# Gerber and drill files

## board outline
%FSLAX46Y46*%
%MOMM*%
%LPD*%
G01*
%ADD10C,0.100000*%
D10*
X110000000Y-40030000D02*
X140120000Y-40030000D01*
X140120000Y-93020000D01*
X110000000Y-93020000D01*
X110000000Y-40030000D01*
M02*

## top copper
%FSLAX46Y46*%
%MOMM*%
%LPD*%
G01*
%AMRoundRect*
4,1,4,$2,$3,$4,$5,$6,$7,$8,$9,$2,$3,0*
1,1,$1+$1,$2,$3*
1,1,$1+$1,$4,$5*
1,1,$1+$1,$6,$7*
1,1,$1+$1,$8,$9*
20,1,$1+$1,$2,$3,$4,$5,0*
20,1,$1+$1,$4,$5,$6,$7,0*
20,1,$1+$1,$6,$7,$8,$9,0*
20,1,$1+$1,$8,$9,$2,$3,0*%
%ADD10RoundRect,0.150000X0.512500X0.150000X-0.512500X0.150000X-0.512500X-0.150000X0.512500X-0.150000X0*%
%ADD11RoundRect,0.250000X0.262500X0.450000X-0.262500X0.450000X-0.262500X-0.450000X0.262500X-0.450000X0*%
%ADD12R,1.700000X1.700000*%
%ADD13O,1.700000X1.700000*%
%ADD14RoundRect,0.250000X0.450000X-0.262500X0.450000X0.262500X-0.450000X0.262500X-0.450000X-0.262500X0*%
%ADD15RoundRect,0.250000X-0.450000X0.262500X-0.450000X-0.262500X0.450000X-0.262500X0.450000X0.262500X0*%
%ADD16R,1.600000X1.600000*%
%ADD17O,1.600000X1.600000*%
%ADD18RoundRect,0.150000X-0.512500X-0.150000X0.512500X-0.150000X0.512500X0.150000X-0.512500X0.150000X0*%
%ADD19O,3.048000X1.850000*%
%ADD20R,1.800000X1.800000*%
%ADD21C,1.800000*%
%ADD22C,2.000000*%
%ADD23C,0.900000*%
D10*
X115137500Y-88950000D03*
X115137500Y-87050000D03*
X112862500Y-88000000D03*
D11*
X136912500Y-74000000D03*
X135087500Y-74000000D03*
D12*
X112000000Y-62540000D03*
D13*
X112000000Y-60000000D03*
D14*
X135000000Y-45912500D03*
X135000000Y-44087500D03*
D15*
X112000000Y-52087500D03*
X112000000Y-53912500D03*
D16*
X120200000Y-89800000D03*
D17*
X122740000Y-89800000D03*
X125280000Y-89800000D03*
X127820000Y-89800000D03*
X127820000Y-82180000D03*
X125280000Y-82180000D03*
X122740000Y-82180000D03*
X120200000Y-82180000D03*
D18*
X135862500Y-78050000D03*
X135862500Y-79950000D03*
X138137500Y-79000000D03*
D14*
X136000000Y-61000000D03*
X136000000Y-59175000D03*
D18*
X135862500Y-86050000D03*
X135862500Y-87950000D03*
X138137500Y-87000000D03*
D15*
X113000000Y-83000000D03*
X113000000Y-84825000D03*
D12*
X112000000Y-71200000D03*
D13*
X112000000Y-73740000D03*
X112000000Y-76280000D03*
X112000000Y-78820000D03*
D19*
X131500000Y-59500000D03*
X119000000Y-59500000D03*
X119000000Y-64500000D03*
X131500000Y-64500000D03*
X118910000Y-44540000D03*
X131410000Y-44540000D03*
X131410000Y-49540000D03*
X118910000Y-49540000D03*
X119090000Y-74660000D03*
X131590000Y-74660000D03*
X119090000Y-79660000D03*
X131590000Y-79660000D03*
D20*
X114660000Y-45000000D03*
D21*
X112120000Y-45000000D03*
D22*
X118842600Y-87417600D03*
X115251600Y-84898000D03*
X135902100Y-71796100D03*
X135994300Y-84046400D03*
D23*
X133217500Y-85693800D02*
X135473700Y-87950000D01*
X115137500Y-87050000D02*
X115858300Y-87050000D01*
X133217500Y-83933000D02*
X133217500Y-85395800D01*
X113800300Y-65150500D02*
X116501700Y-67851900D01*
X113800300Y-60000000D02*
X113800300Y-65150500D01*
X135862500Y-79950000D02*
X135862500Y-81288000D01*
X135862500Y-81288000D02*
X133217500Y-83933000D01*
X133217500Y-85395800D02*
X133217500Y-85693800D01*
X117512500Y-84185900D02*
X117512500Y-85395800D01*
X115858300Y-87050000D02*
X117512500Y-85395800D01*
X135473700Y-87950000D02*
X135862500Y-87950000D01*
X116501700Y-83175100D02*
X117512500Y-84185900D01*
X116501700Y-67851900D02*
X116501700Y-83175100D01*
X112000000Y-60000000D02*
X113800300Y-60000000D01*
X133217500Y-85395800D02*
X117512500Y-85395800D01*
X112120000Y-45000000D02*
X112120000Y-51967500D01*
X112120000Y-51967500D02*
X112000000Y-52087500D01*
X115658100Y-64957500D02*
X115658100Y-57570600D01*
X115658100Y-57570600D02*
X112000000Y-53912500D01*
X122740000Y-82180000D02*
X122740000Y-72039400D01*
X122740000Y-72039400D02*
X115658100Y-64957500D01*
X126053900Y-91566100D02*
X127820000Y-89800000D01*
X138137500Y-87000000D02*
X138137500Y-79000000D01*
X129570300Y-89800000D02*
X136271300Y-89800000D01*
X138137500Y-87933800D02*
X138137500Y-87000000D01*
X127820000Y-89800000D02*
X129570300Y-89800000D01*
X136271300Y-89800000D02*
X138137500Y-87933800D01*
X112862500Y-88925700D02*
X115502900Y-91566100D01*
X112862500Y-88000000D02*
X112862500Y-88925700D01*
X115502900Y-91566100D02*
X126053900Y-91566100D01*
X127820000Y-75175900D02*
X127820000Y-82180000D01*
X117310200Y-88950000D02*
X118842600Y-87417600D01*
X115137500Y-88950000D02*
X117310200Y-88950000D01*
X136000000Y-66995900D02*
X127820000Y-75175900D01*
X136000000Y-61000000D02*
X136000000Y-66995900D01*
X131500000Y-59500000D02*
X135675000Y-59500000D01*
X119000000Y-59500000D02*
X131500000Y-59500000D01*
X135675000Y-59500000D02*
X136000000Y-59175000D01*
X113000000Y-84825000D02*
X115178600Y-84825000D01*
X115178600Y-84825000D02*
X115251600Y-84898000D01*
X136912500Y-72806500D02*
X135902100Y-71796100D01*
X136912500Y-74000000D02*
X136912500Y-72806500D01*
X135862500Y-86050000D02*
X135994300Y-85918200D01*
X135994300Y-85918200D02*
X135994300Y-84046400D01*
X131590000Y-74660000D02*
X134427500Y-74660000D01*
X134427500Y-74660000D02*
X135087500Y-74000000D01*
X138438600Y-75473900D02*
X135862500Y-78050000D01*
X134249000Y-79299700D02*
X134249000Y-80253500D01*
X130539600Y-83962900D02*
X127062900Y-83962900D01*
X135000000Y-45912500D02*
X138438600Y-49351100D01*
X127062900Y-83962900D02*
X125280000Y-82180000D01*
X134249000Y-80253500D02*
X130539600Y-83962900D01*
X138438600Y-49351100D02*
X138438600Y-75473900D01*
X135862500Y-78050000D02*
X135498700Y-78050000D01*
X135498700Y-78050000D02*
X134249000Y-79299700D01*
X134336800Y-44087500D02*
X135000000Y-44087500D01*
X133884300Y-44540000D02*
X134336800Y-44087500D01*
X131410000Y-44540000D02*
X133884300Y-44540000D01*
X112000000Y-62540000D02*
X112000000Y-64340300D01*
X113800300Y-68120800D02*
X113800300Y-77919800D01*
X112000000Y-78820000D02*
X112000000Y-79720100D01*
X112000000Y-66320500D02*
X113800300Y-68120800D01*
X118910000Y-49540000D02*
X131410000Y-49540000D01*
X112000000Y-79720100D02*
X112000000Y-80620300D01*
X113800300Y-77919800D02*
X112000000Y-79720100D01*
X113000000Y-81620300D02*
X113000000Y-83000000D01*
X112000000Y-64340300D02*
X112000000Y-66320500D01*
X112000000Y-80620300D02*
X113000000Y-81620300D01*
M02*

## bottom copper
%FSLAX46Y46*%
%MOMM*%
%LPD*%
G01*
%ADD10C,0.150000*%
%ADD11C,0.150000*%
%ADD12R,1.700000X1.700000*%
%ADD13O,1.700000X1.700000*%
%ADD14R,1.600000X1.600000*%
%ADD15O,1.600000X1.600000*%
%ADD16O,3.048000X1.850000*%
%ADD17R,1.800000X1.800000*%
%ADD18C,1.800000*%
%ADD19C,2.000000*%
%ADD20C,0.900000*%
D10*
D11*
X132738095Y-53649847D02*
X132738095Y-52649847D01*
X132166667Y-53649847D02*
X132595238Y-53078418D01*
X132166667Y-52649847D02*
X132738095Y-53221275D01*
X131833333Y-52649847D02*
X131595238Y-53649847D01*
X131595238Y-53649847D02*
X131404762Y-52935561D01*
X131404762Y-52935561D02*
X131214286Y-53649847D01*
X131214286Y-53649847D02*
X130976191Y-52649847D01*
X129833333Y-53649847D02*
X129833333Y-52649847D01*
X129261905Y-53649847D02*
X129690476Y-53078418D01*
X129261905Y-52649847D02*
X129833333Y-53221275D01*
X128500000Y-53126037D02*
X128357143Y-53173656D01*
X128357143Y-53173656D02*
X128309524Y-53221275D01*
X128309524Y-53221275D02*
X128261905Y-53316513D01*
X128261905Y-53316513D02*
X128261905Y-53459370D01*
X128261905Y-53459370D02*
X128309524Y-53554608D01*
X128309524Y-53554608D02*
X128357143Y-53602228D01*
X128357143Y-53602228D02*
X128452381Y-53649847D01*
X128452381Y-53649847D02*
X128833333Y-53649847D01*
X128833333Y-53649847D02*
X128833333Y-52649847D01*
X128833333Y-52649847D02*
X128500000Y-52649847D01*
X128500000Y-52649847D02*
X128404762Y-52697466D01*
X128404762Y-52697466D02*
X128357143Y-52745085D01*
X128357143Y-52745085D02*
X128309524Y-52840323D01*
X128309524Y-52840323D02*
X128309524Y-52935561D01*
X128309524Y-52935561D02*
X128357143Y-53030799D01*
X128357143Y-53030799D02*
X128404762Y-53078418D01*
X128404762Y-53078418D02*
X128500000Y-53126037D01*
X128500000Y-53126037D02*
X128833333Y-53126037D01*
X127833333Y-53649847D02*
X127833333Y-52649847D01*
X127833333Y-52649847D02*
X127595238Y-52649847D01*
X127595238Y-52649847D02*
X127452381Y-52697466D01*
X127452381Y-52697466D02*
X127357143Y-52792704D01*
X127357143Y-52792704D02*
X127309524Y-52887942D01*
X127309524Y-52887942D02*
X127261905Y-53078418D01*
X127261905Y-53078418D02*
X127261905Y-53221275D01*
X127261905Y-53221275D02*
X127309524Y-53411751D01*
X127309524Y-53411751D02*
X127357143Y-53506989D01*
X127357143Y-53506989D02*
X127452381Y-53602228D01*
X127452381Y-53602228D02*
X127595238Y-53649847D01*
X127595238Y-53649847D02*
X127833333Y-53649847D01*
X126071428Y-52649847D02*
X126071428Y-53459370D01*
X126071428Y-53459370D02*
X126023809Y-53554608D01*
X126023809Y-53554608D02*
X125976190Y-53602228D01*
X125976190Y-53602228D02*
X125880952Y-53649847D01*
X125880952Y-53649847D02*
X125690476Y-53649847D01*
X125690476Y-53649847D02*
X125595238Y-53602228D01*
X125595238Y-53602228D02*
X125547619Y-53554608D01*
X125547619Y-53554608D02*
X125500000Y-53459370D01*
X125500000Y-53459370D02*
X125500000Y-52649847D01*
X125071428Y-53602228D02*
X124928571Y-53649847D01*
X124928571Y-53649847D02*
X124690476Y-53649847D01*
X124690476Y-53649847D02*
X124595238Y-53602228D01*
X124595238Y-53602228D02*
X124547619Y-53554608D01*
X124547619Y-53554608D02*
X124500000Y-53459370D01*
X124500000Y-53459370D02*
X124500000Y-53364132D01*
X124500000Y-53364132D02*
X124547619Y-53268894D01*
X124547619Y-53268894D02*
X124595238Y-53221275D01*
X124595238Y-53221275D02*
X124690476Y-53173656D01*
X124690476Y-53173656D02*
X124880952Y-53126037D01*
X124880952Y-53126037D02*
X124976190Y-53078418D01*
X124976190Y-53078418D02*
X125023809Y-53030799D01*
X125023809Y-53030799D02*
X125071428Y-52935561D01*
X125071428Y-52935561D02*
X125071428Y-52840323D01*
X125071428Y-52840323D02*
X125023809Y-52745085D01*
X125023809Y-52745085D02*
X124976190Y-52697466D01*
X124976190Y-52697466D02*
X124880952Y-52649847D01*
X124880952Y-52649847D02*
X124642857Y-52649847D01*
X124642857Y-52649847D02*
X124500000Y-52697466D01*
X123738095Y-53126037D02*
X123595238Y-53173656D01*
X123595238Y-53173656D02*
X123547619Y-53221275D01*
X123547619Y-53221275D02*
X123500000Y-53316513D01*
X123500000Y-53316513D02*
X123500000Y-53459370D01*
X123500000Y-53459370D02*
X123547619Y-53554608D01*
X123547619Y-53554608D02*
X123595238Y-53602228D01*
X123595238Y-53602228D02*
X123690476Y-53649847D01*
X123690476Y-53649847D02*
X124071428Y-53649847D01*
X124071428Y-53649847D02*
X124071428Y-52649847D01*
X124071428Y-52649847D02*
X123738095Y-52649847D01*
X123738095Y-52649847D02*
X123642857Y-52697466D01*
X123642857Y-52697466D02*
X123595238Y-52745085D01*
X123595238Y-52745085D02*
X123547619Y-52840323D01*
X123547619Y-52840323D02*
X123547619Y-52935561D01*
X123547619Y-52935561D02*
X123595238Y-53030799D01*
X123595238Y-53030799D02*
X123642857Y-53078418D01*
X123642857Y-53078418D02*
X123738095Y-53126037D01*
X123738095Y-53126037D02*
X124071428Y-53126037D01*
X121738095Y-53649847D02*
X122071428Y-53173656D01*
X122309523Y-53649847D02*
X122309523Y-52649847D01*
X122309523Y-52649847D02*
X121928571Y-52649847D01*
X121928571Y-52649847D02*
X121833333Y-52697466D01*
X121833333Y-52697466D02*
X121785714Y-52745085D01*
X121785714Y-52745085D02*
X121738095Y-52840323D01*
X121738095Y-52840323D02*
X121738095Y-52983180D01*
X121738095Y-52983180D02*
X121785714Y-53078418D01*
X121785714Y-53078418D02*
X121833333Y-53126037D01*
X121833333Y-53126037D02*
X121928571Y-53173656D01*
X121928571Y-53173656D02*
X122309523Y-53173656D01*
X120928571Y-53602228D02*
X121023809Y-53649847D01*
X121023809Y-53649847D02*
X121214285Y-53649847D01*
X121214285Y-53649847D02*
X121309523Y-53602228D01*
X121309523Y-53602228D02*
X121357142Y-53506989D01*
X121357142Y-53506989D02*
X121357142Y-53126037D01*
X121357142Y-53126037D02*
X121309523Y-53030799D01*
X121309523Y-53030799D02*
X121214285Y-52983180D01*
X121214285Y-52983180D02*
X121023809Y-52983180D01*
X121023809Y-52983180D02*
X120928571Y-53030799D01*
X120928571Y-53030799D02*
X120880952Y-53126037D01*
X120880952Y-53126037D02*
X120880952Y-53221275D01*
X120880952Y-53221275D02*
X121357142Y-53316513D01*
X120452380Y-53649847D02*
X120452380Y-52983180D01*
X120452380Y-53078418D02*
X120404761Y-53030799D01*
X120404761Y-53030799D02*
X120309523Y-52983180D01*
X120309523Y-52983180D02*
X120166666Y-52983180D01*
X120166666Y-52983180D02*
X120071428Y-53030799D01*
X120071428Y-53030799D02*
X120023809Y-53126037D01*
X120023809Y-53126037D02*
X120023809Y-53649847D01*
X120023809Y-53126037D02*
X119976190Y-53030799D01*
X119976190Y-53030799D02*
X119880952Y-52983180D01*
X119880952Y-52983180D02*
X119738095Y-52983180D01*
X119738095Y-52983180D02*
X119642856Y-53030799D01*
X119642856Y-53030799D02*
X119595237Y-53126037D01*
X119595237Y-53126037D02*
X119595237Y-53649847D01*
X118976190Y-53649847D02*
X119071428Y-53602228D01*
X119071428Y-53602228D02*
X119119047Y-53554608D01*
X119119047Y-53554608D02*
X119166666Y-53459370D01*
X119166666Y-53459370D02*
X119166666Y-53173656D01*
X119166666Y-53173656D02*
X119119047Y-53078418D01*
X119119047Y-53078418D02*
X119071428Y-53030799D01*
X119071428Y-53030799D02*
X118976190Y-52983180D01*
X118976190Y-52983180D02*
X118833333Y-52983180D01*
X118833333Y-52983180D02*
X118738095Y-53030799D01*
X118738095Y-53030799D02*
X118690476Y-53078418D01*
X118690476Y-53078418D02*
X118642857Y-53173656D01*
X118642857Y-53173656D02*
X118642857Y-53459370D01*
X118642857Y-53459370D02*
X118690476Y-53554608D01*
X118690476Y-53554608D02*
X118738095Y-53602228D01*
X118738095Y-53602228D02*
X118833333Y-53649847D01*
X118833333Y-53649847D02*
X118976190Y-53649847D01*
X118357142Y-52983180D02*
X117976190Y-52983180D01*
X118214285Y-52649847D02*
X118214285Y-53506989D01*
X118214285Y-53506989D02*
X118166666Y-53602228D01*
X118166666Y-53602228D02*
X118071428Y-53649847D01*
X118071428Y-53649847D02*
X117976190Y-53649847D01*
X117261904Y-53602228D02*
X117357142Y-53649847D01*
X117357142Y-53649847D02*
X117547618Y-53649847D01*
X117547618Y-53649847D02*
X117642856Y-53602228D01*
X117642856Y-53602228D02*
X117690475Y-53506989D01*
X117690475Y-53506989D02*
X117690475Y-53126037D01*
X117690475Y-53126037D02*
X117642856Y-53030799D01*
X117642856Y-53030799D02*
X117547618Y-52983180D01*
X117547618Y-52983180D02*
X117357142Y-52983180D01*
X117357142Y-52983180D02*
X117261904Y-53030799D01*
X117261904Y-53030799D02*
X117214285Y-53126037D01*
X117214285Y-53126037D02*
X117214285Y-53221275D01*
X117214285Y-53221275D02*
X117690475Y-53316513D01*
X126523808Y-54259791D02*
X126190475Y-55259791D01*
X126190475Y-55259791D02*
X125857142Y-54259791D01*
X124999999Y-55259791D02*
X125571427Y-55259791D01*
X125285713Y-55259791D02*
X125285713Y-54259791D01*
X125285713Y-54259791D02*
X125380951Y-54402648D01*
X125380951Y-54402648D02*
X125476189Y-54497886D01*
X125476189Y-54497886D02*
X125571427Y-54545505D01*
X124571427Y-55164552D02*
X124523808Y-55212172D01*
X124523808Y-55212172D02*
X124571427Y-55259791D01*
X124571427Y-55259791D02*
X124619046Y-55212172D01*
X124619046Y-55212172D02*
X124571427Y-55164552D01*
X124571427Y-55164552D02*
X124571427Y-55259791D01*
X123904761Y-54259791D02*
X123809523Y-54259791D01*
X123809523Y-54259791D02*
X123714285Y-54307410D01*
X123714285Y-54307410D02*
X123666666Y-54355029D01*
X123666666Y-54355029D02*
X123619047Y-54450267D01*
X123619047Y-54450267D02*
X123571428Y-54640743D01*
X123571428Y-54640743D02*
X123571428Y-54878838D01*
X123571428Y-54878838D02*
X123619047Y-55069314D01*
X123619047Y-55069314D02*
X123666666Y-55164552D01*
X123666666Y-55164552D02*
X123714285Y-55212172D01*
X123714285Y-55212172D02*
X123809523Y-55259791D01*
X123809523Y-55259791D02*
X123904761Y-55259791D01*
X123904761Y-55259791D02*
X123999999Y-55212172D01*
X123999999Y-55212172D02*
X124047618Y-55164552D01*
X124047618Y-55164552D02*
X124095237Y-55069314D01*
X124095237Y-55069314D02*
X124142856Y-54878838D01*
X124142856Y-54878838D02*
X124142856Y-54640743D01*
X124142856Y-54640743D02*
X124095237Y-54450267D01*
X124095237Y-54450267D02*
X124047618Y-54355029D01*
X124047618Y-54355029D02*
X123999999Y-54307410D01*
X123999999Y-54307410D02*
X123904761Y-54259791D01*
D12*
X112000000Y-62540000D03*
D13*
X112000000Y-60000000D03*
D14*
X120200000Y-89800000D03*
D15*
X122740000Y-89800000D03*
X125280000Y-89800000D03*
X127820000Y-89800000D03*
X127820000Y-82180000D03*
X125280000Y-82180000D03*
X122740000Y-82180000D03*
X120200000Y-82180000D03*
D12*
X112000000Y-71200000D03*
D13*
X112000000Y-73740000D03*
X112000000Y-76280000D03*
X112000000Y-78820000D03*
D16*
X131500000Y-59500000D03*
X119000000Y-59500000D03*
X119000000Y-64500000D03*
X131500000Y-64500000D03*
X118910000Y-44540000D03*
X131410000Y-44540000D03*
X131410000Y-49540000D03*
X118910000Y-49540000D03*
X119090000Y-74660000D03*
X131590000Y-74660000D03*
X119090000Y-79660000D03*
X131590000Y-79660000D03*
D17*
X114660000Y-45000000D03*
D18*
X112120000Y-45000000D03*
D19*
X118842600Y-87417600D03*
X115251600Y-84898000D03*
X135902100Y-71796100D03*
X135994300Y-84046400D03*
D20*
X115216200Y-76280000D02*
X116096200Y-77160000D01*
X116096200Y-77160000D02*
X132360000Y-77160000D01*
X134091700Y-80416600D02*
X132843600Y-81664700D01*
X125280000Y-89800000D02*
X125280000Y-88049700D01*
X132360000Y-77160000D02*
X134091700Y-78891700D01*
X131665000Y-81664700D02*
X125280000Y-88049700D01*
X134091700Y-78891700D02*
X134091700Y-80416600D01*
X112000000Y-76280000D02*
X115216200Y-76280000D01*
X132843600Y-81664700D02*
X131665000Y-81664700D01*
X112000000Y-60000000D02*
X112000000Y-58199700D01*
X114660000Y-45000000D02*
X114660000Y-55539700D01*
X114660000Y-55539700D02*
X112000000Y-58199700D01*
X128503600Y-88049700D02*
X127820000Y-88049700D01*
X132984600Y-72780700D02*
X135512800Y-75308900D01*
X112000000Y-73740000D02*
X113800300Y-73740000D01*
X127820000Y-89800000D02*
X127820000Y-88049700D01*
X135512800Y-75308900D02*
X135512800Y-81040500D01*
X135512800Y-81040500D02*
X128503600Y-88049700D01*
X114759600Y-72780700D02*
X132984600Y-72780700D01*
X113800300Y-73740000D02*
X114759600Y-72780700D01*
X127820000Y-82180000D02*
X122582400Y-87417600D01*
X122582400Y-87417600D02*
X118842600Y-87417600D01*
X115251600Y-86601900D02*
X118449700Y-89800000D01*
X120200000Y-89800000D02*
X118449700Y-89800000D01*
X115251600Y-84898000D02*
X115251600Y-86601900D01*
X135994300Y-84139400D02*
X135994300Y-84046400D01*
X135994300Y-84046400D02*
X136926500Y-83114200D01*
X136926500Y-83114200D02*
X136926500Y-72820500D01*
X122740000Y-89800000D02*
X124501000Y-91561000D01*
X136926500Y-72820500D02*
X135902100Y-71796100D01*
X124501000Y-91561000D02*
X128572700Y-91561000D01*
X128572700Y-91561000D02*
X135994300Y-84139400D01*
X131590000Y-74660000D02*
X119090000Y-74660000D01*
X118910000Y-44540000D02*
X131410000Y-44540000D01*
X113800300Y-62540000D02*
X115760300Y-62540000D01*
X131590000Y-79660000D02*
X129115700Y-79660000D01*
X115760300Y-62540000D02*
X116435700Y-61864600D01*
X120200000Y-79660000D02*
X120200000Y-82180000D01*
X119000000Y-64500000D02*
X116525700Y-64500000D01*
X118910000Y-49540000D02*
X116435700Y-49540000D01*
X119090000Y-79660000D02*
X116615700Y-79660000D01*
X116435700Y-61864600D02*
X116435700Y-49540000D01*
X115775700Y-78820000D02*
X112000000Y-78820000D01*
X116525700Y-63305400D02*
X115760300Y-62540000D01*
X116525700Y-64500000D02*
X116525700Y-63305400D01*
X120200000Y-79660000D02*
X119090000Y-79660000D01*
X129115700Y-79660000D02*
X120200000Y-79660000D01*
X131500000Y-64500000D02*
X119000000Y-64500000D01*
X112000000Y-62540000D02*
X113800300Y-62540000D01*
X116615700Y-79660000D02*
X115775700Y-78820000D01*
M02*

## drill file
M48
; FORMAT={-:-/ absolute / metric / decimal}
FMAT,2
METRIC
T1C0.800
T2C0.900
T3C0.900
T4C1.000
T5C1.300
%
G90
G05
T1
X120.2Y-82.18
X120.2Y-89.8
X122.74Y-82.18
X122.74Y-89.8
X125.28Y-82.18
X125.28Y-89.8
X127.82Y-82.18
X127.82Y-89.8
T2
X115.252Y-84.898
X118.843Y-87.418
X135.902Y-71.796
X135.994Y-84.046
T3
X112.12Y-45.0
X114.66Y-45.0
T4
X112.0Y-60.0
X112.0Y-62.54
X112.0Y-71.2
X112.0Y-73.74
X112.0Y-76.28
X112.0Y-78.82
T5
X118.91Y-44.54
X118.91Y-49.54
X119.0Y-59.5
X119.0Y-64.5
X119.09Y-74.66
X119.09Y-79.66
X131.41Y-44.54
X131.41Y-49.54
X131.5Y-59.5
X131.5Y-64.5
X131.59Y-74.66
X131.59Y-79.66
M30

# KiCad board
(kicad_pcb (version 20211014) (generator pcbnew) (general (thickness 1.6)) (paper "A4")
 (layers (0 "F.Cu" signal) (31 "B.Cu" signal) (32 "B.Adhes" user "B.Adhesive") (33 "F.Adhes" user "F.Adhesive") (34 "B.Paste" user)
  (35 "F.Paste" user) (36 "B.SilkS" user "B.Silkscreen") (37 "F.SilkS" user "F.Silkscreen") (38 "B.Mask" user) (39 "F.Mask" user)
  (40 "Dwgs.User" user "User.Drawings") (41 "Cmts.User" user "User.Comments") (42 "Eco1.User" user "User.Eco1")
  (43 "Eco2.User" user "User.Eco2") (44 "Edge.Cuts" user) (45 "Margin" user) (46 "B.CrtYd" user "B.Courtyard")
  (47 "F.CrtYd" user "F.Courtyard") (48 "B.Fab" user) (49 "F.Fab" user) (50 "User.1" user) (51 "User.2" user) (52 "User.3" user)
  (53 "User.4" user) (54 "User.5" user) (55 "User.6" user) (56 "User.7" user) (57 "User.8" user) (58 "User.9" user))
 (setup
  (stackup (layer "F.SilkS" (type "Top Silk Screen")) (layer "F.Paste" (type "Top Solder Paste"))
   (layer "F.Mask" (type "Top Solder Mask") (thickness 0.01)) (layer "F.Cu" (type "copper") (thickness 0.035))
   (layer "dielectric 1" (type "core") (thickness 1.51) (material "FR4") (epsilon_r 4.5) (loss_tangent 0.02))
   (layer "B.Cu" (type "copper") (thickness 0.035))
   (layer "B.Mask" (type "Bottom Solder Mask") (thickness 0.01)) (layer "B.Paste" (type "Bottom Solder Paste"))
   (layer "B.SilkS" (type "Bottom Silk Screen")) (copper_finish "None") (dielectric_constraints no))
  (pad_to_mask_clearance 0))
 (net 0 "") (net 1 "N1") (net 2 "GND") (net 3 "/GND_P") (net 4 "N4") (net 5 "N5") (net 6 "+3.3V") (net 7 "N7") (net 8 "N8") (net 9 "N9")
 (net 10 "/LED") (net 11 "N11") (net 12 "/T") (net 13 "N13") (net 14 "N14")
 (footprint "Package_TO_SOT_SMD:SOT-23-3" (layer "F.Cu") (at 114 88 180)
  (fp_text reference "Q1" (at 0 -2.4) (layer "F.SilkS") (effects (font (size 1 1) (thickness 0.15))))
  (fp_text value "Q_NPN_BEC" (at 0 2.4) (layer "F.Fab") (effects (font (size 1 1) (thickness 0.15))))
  (pad "1" smd roundrect locked (at -1.1375 -0.95 180) (size 1.325 0.6) (layers "F.Cu" "F.Paste" "F.Mask") (roundrect_rratio 0.25)
   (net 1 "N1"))
  (pad "2" smd roundrect locked (at -1.1375 0.95 180) (size 1.325 0.6) (layers "F.Cu" "F.Paste" "F.Mask") (roundrect_rratio 0.25)
   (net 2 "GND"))
  (pad "3" smd roundrect locked (at 1.1375 0 180) (size 1.325 0.6) (layers "F.Cu" "F.Paste" "F.Mask") (roundrect_rratio 0.25)
   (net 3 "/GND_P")))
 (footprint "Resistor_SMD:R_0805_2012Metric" (layer "F.Cu") (at 136 74 180)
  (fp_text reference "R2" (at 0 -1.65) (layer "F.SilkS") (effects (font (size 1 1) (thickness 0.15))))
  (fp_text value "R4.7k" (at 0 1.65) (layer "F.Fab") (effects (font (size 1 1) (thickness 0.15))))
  (pad "1" smd roundrect (at -0.9125 0 180) (size 1.025 1.4) (layers "F.Cu" "F.Paste" "F.Mask") (roundrect_rratio 0.243902439) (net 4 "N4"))
  (pad "2" smd roundrect (at 0.9125 0 180) (size 1.025 1.4) (layers "F.Cu" "F.Paste" "F.Mask") (roundrect_rratio 0.243902439) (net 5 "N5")))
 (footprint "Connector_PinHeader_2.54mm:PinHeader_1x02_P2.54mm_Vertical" (layer "F.Cu") (at 112 62.54 180)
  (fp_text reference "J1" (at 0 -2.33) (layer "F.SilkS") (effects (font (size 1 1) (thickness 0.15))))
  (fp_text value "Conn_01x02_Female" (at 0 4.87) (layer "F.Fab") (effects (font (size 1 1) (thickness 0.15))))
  (pad "1" thru_hole rect (at 0 0 180) (size 1.7 1.7) (drill 1) (layers *.Cu *.Mask) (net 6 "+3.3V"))
  (pad "2" thru_hole oval (at 0 2.54 180) (size 1.7 1.7) (drill 1) (layers *.Cu *.Mask) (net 2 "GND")))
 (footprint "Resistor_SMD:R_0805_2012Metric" (layer "F.Cu") (at 135 45 90)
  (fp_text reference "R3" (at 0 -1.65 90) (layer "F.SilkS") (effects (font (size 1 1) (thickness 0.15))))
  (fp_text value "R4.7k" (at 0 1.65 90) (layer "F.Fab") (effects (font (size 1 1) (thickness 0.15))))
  (pad "1" smd roundrect (at -0.9125 0 90) (size 1.025 1.4) (layers "F.Cu" "F.Paste" "F.Mask") (roundrect_rratio 0.243902439) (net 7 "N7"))
  (pad "2" smd roundrect (at 0.9125 0 90) (size 1.025 1.4) (layers "F.Cu" "F.Paste" "F.Mask") (roundrect_rratio 0.243902439) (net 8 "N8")))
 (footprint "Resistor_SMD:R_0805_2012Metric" (layer "F.Cu") (at 112 53 -90)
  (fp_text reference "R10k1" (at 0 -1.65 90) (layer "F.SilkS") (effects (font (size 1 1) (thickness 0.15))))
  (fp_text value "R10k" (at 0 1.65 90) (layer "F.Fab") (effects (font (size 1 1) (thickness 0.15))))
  (pad "1" smd roundrect (at -0.9125 0 270) (size 1.025 1.4) (layers "F.Cu" "F.Paste" "F.Mask") (roundrect_rratio 0.243902439) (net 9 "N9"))
  (pad "2" smd roundrect (at 0.9125 0 270) (size 1.025 1.4) (layers "F.Cu" "F.Paste" "F.Mask") (roundrect_rratio 0.243902439)
   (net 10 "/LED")))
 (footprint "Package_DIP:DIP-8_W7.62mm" (layer "F.Cu") (at 120.2 89.8 90)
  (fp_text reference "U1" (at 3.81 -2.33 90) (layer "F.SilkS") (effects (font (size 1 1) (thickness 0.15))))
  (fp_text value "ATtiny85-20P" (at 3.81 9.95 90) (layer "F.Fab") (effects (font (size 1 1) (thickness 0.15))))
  (pad "1" thru_hole rect (at 0 0 90) (size 1.6 1.6) (drill 0.8) (layers *.Cu *.Mask) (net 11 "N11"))
  (pad "2" thru_hole oval (at 0 2.54 90) (size 1.6 1.6) (drill 0.8) (layers *.Cu *.Mask) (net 4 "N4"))
  (pad "3" thru_hole oval (at 0 5.08 90) (size 1.6 1.6) (drill 0.8) (layers *.Cu *.Mask) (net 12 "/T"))
  (pad "4" thru_hole oval (at 0 7.62 90) (size 1.6 1.6) (drill 0.8) (layers *.Cu *.Mask) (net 3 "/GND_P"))
  (pad "5" thru_hole oval (at 7.62 7.62 90) (size 1.6 1.6) (drill 0.8) (layers *.Cu *.Mask) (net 1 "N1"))
  (pad "6" thru_hole oval (at 7.62 5.08 90) (size 1.6 1.6) (drill 0.8) (layers *.Cu *.Mask) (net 7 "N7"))
  (pad "7" thru_hole oval (at 7.62 2.54 90) (size 1.6 1.6) (drill 0.8) (layers *.Cu *.Mask) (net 10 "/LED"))
  (pad "8" thru_hole oval (at 7.62 0 90) (size 1.6 1.6) (drill 0.8) (layers *.Cu *.Mask) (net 6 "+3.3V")))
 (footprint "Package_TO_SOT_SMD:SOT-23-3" (layer "F.Cu") (at 137 79)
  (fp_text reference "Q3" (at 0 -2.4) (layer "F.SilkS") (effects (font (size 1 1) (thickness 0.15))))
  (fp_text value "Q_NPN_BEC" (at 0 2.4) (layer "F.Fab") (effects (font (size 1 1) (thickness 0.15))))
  (pad "1" smd roundrect locked (at -1.1375 -0.95) (size 1.325 0.6) (layers "F.Cu" "F.Paste" "F.Mask") (roundrect_rratio 0.25) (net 7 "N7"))
  (pad "2" smd roundrect locked (at -1.1375 0.95) (size 1.325 0.6) (layers "F.Cu" "F.Paste" "F.Mask") (roundrect_rratio 0.25) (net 2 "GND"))
  (pad "3" smd roundrect locked (at 1.1375 0) (size 1.325 0.6) (layers "F.Cu" "F.Paste" "F.Mask") (roundrect_rratio 0.25) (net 3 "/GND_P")))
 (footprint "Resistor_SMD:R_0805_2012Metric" (layer "F.Cu") (at 136 60.0875 90)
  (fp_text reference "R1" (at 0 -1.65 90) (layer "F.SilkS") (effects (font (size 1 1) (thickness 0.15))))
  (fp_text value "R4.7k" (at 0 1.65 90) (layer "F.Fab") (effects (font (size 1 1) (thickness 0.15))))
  (pad "1" smd roundrect (at -0.9125 0 90) (size 1.025 1.4) (layers "F.Cu" "F.Paste" "F.Mask") (roundrect_rratio 0.243902439) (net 1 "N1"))
  (pad "2" smd roundrect (at 0.9125 0 90) (size 1.025 1.4) (layers "F.Cu" "F.Paste" "F.Mask") (roundrect_rratio 0.243902439) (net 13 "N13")))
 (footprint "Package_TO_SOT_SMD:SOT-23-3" (layer "F.Cu") (at 137 87)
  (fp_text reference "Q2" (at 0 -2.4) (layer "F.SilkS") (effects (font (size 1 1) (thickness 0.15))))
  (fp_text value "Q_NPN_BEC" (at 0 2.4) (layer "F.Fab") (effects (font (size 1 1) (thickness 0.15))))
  (pad "1" smd roundrect locked (at -1.1375 -0.95) (size 1.325 0.6) (layers "F.Cu" "F.Paste" "F.Mask") (roundrect_rratio 0.25) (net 4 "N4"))
  (pad "2" smd roundrect locked (at -1.1375 0.95) (size 1.325 0.6) (layers "F.Cu" "F.Paste" "F.Mask") (roundrect_rratio 0.25) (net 2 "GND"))
  (pad "3" smd roundrect locked (at 1.1375 0) (size 1.325 0.6) (layers "F.Cu" "F.Paste" "F.Mask") (roundrect_rratio 0.25) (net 3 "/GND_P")))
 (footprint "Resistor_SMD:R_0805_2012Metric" (layer "F.Cu") (at 113 83.9125 -90)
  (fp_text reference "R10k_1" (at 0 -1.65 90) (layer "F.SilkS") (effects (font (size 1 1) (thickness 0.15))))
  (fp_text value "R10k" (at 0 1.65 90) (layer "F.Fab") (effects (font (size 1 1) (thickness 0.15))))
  (pad "1" smd roundrect (at -0.9125 0 270) (size 1.025 1.4) (layers "F.Cu" "F.Paste" "F.Mask") (roundrect_rratio 0.243902439)
   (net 6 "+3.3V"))
  (pad "2" smd roundrect (at 0.9125 0 270) (size 1.025 1.4) (layers "F.Cu" "F.Paste" "F.Mask") (roundrect_rratio 0.243902439) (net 11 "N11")))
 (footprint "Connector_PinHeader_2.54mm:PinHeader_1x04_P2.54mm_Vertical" (layer "F.Cu") (at 112 71.2)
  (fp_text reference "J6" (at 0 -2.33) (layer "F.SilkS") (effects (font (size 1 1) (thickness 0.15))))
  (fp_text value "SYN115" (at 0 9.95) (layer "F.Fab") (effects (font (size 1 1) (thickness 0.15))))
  (pad "1" thru_hole rect (at 0 0) (size 1.7 1.7) (drill 1) (layers *.Cu *.Mask) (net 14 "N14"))
  (pad "2" thru_hole oval (at 0 2.54) (size 1.7 1.7) (drill 1) (layers *.Cu *.Mask) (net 3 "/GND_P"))
  (pad "3" thru_hole oval (at 0 5.08) (size 1.7 1.7) (drill 1) (layers *.Cu *.Mask) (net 12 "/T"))
  (pad "4" thru_hole oval (at 0 7.62) (size 1.7 1.7) (drill 1) (layers *.Cu *.Mask) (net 6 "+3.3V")))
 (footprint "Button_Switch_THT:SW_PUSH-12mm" (layer "B.Cu") (at 131.5 59.5 180)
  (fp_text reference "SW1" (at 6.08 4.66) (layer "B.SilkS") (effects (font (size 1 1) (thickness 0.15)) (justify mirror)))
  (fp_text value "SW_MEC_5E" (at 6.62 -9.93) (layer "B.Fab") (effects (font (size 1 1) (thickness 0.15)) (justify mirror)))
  (pad "1" thru_hole oval (at 0 0 180) (size 3.048 1.85) (drill 1.3) (layers *.Cu *.Mask) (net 13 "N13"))
  (pad "1" thru_hole oval (at 12.5 0 180) (size 3.048 1.85) (drill 1.3) (layers *.Cu *.Mask) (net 13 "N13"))
  (pad "2" thru_hole oval (at 12.5 -5 180) (size 3.048 1.85) (drill 1.3) (layers *.Cu *.Mask) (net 6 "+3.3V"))
  (pad "2" thru_hole oval (at 0 -5 180) (size 3.048 1.85) (drill 1.3) (layers *.Cu *.Mask) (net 6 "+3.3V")))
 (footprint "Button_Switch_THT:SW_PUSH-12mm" (layer "B.Cu") (at 131.41 44.54 180)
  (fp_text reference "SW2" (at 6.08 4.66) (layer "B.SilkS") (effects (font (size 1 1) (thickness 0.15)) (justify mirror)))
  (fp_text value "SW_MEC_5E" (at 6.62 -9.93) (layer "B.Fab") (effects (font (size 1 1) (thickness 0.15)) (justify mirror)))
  (pad "1" thru_hole oval (at 12.5 0 180) (size 3.048 1.85) (drill 1.3) (layers *.Cu *.Mask) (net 8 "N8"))
  (pad "1" thru_hole oval (at 0 0 180) (size 3.048 1.85) (drill 1.3) (layers *.Cu *.Mask) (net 8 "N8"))
  (pad "2" thru_hole oval (at 0 -5 180) (size 3.048 1.85) (drill 1.3) (layers *.Cu *.Mask) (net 6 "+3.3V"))
  (pad "2" thru_hole oval (at 12.5 -5 180) (size 3.048 1.85) (drill 1.3) (layers *.Cu *.Mask) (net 6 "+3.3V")))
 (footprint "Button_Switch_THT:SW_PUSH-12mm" (layer "B.Cu") (at 131.59 74.66 180)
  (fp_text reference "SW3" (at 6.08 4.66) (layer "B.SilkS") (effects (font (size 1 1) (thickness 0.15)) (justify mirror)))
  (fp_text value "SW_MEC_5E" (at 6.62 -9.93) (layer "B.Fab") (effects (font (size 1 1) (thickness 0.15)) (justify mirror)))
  (pad "1" thru_hole oval (at 12.5 0 180) (size 3.048 1.85) (drill 1.3) (layers *.Cu *.Mask) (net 5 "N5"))
  (pad "1" thru_hole oval (at 0 0 180) (size 3.048 1.85) (drill 1.3) (layers *.Cu *.Mask) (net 5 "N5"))
  (pad "2" thru_hole oval (at 12.5 -5 180) (size 3.048 1.85) (drill 1.3) (layers *.Cu *.Mask) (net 6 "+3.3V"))
  (pad "2" thru_hole oval (at 0 -5 180) (size 3.048 1.85) (drill 1.3) (layers *.Cu *.Mask) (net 6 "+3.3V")))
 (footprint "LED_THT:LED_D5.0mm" (layer "B.Cu") (at 114.66 45 180)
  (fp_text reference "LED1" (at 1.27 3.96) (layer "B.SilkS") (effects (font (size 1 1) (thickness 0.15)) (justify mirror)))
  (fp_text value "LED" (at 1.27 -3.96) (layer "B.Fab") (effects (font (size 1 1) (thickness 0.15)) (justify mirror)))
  (pad "1" thru_hole rect (at 0 0 180) (size 1.8 1.8) (drill 0.9) (layers *.Cu *.Mask) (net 2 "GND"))
  (pad "2" thru_hole circle (at 2.54 0 180) (size 1.8 1.8) (drill 0.9) (layers *.Cu *.Mask) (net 9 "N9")))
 (gr_rect (start 140.12 93.02) (end 110 40.03) (layer "Edge.Cuts") (width 0.1) (fill none))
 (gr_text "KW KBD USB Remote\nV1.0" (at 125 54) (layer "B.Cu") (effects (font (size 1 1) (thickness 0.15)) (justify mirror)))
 (segment (start 115.2162 76.28) (end 116.0962 77.16) (width 0.9) (layer "B.Cu") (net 12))
 (segment (start 116.0962 77.16) (end 132.36 77.16) (width 0.9) (layer "B.Cu") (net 12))
 (segment (start 134.0917 80.4166) (end 132.8436 81.6647) (width 0.9) (layer "B.Cu") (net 12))
 (segment (start 125.28 89.8) (end 125.28 88.0497) (width 0.9) (layer "B.Cu") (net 12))
 (segment (start 132.36 77.16) (end 134.0917 78.8917) (width 0.9) (layer "B.Cu") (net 12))
 (segment (start 131.665 81.6647) (end 125.28 88.0497) (width 0.9) (layer "B.Cu") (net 12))
 (segment (start 134.0917 78.8917) (end 134.0917 80.4166) (width 0.9) (layer "B.Cu") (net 12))
 (segment (start 112 76.28) (end 115.2162 76.28) (width 0.9) (layer "B.Cu") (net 12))
 (segment (start 132.8436 81.6647) (end 131.665 81.6647) (width 0.9) (layer "B.Cu") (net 12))
 (segment (start 133.2175 85.6938) (end 135.4737 87.95) (width 0.9) (layer "F.Cu") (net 2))
 (segment (start 115.1375 87.05) (end 115.8583 87.05) (width 0.9) (layer "F.Cu") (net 2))
 (segment (start 133.2175 83.933) (end 133.2175 85.3958) (width 0.9) (layer "F.Cu") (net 2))
 (segment (start 113.8003 65.1505) (end 116.5017 67.8519) (width 0.9) (layer "F.Cu") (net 2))
 (segment (start 113.8003 60) (end 113.8003 65.1505) (width 0.9) (layer "F.Cu") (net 2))
 (segment (start 135.8625 79.95) (end 135.8625 81.288) (width 0.9) (layer "F.Cu") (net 2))
 (segment (start 135.8625 81.288) (end 133.2175 83.933) (width 0.9) (layer "F.Cu") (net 2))
 (segment (start 133.2175 85.3958) (end 133.2175 85.6938) (width 0.9) (layer "F.Cu") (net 2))
 (segment (start 117.5125 84.1859) (end 117.5125 85.3958) (width 0.9) (layer "F.Cu") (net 2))
 (segment (start 115.8583 87.05) (end 117.5125 85.3958) (width 0.9) (layer "F.Cu") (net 2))
 (segment (start 135.4737 87.95) (end 135.8625 87.95) (width 0.9) (layer "F.Cu") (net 2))
 (segment (start 116.5017 83.1751) (end 117.5125 84.1859) (width 0.9) (layer "F.Cu") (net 2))
 (segment (start 116.5017 67.8519) (end 116.5017 83.1751) (width 0.9) (layer "F.Cu") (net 2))
 (segment (start 112 60) (end 113.8003 60) (width 0.9) (layer "F.Cu") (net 2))
 (segment (start 133.2175 85.3958) (end 117.5125 85.3958) (width 0.9) (layer "F.Cu") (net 2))
 (segment (start 112 60) (end 112 58.1997) (width 0.9) (layer "B.Cu") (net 2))
 (segment (start 114.66 45) (end 114.66 55.5397) (width 0.9) (layer "B.Cu") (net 2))
 (segment (start 114.66 55.5397) (end 112 58.1997) (width 0.9) (layer "B.Cu") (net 2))
 (segment (start 112.12 45) (end 112.12 51.9675) (width 0.9) (layer "F.Cu") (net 9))
 (segment (start 112.12 51.9675) (end 112 52.0875) (width 0.9) (layer "F.Cu") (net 9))
 (segment (start 115.6581 64.9575) (end 115.6581 57.5706) (width 0.9) (layer "F.Cu") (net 10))
 (segment (start 115.6581 57.5706) (end 112 53.9125) (width 0.9) (layer "F.Cu") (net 10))
 (segment (start 122.74 82.18) (end 122.74 72.0394) (width 0.9) (layer "F.Cu") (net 10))
 (segment (start 122.74 72.0394) (end 115.6581 64.9575) (width 0.9) (layer "F.Cu") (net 10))
 (segment (start 126.0539 91.5661) (end 127.82 89.8) (width 0.9) (layer "F.Cu") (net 3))
 (segment (start 138.1375 87) (end 138.1375 79) (width 0.9) (layer "F.Cu") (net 3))
 (segment (start 129.5703 89.8) (end 136.2713 89.8) (width 0.9) (layer "F.Cu") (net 3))
 (segment (start 138.1375 87.9338) (end 138.1375 87) (width 0.9) (layer "F.Cu") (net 3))
 (segment (start 127.82 89.8) (end 129.5703 89.8) (width 0.9) (layer "F.Cu") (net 3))
 (segment (start 136.2713 89.8) (end 138.1375 87.9338) (width 0.9) (layer "F.Cu") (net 3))
 (segment (start 112.8625 88.9257) (end 115.5029 91.5661) (width 0.9) (layer "F.Cu") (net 3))
 (segment (start 112.8625 88) (end 112.8625 88.9257) (width 0.9) (layer "F.Cu") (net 3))
 (segment (start 115.5029 91.5661) (end 126.0539 91.5661) (width 0.9) (layer "F.Cu") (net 3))
 (segment (start 128.5036 88.0497) (end 127.82 88.0497) (width 0.9) (layer "B.Cu") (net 3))
 (segment (start 132.9846 72.7807) (end 135.5128 75.3089) (width 0.9) (layer "B.Cu") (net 3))
 (segment (start 112 73.74) (end 113.8003 73.74) (width 0.9) (layer "B.Cu") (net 3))
 (segment (start 127.82 89.8) (end 127.82 88.0497) (width 0.9) (layer "B.Cu") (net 3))
 (segment (start 135.5128 75.3089) (end 135.5128 81.0405) (width 0.9) (layer "B.Cu") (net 3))
 (segment (start 135.5128 81.0405) (end 128.5036 88.0497) (width 0.9) (layer "B.Cu") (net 3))
 (segment (start 114.7596 72.7807) (end 132.9846 72.7807) (width 0.9) (layer "B.Cu") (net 3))
 (segment (start 113.8003 73.74) (end 114.7596 72.7807) (width 0.9) (layer "B.Cu") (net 3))
 (segment (start 127.82 75.1759) (end 127.82 82.18) (width 0.9) (layer "F.Cu") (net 1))
 (segment (start 117.3102 88.95) (end 118.8426 87.4176) (width 0.9) (layer "F.Cu") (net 1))
 (segment (start 115.1375 88.95) (end 117.3102 88.95) (width 0.9) (layer "F.Cu") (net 1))
 (segment (start 136 66.9959) (end 127.82 75.1759) (width 0.9) (layer "F.Cu") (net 1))
 (segment (start 136 61) (end 136 66.9959) (width 0.9) (layer "F.Cu") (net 1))
 (via (at 118.8426 87.4176) (size 2) (drill 0.9) (layers "F.Cu" "B.Cu") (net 1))
 (segment (start 127.82 82.18) (end 122.5824 87.4176) (width 0.9) (layer "B.Cu") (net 1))
 (segment (start 122.5824 87.4176) (end 118.8426 87.4176) (width 0.9) (layer "B.Cu") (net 1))
 (segment (start 131.5 59.5) (end 135.675 59.5) (width 0.9) (layer "F.Cu") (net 13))
 (segment (start 119 59.5) (end 131.5 59.5) (width 0.9) (layer "F.Cu") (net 13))
 (segment (start 135.675 59.5) (end 136 59.175) (width 0.9) (layer "F.Cu") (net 13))
 (segment (start 113 84.825) (end 115.1786 84.825) (width 0.9) (layer "F.Cu") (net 11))
 (segment (start 115.1786 84.825) (end 115.2516 84.898) (width 0.9) (layer "F.Cu") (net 11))
 (via (at 115.2516 84.898) (size 2) (drill 0.9) (layers "F.Cu" "B.Cu") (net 11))
 (segment (start 115.2516 86.6019) (end 118.4497 89.8) (width 0.9) (layer "B.Cu") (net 11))
 (segment (start 120.2 89.8) (end 118.4497 89.8) (width 0.9) (layer "B.Cu") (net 11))
 (segment (start 115.2516 84.898) (end 115.2516 86.6019) (width 0.9) (layer "B.Cu") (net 11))
 (segment (start 136.9125 72.8065) (end 135.9021 71.7961) (width 0.9) (layer "F.Cu") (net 4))
 (segment (start 136.9125 74) (end 136.9125 72.8065) (width 0.9) (layer "F.Cu") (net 4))
 (segment (start 135.8625 86.05) (end 135.9943 85.9182) (width 0.9) (layer "F.Cu") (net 4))
 (segment (start 135.9943 85.9182) (end 135.9943 84.0464) (width 0.9) (layer "F.Cu") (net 4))
 (via (at 135.9021 71.7961) (size 2) (drill 0.9) (layers "F.Cu" "B.Cu") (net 4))
 (via (at 135.9943 84.0464) (size 2) (drill 0.9) (layers "F.Cu" "B.Cu") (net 4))
 (segment (start 135.9943 84.1394) (end 135.9943 84.0464) (width 0.9) (layer "B.Cu") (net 4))
 (segment (start 135.9943 84.0464) (end 136.9265 83.1142) (width 0.9) (layer "B.Cu") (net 4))
 (segment (start 136.9265 83.1142) (end 136.9265 72.8205) (width 0.9) (layer "B.Cu") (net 4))
 (segment (start 122.74 89.8) (end 124.501 91.561) (width 0.9) (layer "B.Cu") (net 4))
 (segment (start 136.9265 72.8205) (end 135.9021 71.7961) (width 0.9) (layer "B.Cu") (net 4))
 (segment (start 124.501 91.561) (end 128.5727 91.561) (width 0.9) (layer "B.Cu") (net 4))
 (segment (start 128.5727 91.561) (end 135.9943 84.1394) (width 0.9) (layer "B.Cu") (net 4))
 (segment (start 131.59 74.66) (end 134.4275 74.66) (width 0.9) (layer "F.Cu") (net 5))
 (segment (start 134.4275 74.66) (end 135.0875 74) (width 0.9) (layer "F.Cu") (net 5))
 (segment (start 131.59 74.66) (end 119.09 74.66) (width 0.9) (layer "B.Cu") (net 5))
 (segment (start 138.4386 75.4739) (end 135.8625 78.05) (width 0.9) (layer "F.Cu") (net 7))
 (segment (start 134.249 79.2997) (end 134.249 80.2535) (width 0.9) (layer "F.Cu") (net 7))
 (segment (start 130.5396 83.9629) (end 127.0629 83.9629) (width 0.9) (layer "F.Cu") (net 7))
 (segment (start 135 45.9125) (end 138.4386 49.3511) (width 0.9) (layer "F.Cu") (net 7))
 (segment (start 127.0629 83.9629) (end 125.28 82.18) (width 0.9) (layer "F.Cu") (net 7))
 (segment (start 134.249 80.2535) (end 130.5396 83.9629) (width 0.9) (layer "F.Cu") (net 7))
 (segment (start 138.4386 49.3511) (end 138.4386 75.4739) (width 0.9) (layer "F.Cu") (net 7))
 (segment (start 135.8625 78.05) (end 135.4987 78.05) (width 0.9) (layer "F.Cu") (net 7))
 (segment (start 135.4987 78.05) (end 134.249 79.2997) (width 0.9) (layer "F.Cu") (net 7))
 (segment (start 134.3368 44.0875) (end 135 44.0875) (width 0.9) (layer "F.Cu") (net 8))
 (segment (start 133.8843 44.54) (end 134.3368 44.0875) (width 0.9) (layer "F.Cu") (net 8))
 (segment (start 131.41 44.54) (end 133.8843 44.54) (width 0.9) (layer "F.Cu") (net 8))
 (segment (start 118.91 44.54) (end 131.41 44.54) (width 0.9) (layer "B.Cu") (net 8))
 (segment (start 112 62.54) (end 112 64.3403) (width 0.9) (layer "F.Cu") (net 6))
 (segment (start 113.8003 68.1208) (end 113.8003 77.9198) (width 0.9) (layer "F.Cu") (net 6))
 (segment (start 112 78.82) (end 112 79.7201) (width 0.9) (layer "F.Cu") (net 6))
 (segment (start 112 66.3205) (end 113.8003 68.1208) (width 0.9) (layer "F.Cu") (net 6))
 (segment (start 118.91 49.54) (end 131.41 49.54) (width 0.9) (layer "F.Cu") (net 6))
 (segment (start 112 79.7201) (end 112 80.6203) (width 0.9) (layer "F.Cu") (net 6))
 (segment (start 113.8003 77.9198) (end 112 79.7201) (width 0.9) (layer "F.Cu") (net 6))
 (segment (start 113 81.6203) (end 113 83) (width 0.9) (layer "F.Cu") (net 6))
 (segment (start 112 64.3403) (end 112 66.3205) (width 0.9) (layer "F.Cu") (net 6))
 (segment (start 112 80.6203) (end 113 81.6203) (width 0.9) (layer "F.Cu") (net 6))
 (segment (start 113.8003 62.54) (end 115.7603 62.54) (width 0.9) (layer "B.Cu") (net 6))
 (segment (start 131.59 79.66) (end 129.1157 79.66) (width 0.9) (layer "B.Cu") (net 6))
 (segment (start 115.7603 62.54) (end 116.4357 61.8646) (width 0.9) (layer "B.Cu") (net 6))
 (segment (start 120.2 79.66) (end 120.2 82.18) (width 0.9) (layer "B.Cu") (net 6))
 (segment (start 119 64.5) (end 116.5257 64.5) (width 0.9) (layer "B.Cu") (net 6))
 (segment (start 118.91 49.54) (end 116.4357 49.54) (width 0.9) (layer "B.Cu") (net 6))
 (segment (start 119.09 79.66) (end 116.6157 79.66) (width 0.9) (layer "B.Cu") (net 6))
 (segment (start 116.4357 61.8646) (end 116.4357 49.54) (width 0.9) (layer "B.Cu") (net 6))
 (segment (start 115.7757 78.82) (end 112 78.82) (width 0.9) (layer "B.Cu") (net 6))
 (segment (start 116.5257 63.3054) (end 115.7603 62.54) (width 0.9) (layer "B.Cu") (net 6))
 (segment (start 116.5257 64.5) (end 116.5257 63.3054) (width 0.9) (layer "B.Cu") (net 6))
 (segment (start 120.2 79.66) (end 119.09 79.66) (width 0.9) (layer "B.Cu") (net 6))
 (segment (start 129.1157 79.66) (end 120.2 79.66) (width 0.9) (layer "B.Cu") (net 6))
 (segment (start 131.5 64.5) (end 119 64.5) (width 0.9) (layer "B.Cu") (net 6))
 (segment (start 112 62.54) (end 113.8003 62.54) (width 0.9) (layer "B.Cu") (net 6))
 (segment (start 116.6157 79.66) (end 115.7757 78.82) (width 0.9) (layer "B.Cu") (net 6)))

